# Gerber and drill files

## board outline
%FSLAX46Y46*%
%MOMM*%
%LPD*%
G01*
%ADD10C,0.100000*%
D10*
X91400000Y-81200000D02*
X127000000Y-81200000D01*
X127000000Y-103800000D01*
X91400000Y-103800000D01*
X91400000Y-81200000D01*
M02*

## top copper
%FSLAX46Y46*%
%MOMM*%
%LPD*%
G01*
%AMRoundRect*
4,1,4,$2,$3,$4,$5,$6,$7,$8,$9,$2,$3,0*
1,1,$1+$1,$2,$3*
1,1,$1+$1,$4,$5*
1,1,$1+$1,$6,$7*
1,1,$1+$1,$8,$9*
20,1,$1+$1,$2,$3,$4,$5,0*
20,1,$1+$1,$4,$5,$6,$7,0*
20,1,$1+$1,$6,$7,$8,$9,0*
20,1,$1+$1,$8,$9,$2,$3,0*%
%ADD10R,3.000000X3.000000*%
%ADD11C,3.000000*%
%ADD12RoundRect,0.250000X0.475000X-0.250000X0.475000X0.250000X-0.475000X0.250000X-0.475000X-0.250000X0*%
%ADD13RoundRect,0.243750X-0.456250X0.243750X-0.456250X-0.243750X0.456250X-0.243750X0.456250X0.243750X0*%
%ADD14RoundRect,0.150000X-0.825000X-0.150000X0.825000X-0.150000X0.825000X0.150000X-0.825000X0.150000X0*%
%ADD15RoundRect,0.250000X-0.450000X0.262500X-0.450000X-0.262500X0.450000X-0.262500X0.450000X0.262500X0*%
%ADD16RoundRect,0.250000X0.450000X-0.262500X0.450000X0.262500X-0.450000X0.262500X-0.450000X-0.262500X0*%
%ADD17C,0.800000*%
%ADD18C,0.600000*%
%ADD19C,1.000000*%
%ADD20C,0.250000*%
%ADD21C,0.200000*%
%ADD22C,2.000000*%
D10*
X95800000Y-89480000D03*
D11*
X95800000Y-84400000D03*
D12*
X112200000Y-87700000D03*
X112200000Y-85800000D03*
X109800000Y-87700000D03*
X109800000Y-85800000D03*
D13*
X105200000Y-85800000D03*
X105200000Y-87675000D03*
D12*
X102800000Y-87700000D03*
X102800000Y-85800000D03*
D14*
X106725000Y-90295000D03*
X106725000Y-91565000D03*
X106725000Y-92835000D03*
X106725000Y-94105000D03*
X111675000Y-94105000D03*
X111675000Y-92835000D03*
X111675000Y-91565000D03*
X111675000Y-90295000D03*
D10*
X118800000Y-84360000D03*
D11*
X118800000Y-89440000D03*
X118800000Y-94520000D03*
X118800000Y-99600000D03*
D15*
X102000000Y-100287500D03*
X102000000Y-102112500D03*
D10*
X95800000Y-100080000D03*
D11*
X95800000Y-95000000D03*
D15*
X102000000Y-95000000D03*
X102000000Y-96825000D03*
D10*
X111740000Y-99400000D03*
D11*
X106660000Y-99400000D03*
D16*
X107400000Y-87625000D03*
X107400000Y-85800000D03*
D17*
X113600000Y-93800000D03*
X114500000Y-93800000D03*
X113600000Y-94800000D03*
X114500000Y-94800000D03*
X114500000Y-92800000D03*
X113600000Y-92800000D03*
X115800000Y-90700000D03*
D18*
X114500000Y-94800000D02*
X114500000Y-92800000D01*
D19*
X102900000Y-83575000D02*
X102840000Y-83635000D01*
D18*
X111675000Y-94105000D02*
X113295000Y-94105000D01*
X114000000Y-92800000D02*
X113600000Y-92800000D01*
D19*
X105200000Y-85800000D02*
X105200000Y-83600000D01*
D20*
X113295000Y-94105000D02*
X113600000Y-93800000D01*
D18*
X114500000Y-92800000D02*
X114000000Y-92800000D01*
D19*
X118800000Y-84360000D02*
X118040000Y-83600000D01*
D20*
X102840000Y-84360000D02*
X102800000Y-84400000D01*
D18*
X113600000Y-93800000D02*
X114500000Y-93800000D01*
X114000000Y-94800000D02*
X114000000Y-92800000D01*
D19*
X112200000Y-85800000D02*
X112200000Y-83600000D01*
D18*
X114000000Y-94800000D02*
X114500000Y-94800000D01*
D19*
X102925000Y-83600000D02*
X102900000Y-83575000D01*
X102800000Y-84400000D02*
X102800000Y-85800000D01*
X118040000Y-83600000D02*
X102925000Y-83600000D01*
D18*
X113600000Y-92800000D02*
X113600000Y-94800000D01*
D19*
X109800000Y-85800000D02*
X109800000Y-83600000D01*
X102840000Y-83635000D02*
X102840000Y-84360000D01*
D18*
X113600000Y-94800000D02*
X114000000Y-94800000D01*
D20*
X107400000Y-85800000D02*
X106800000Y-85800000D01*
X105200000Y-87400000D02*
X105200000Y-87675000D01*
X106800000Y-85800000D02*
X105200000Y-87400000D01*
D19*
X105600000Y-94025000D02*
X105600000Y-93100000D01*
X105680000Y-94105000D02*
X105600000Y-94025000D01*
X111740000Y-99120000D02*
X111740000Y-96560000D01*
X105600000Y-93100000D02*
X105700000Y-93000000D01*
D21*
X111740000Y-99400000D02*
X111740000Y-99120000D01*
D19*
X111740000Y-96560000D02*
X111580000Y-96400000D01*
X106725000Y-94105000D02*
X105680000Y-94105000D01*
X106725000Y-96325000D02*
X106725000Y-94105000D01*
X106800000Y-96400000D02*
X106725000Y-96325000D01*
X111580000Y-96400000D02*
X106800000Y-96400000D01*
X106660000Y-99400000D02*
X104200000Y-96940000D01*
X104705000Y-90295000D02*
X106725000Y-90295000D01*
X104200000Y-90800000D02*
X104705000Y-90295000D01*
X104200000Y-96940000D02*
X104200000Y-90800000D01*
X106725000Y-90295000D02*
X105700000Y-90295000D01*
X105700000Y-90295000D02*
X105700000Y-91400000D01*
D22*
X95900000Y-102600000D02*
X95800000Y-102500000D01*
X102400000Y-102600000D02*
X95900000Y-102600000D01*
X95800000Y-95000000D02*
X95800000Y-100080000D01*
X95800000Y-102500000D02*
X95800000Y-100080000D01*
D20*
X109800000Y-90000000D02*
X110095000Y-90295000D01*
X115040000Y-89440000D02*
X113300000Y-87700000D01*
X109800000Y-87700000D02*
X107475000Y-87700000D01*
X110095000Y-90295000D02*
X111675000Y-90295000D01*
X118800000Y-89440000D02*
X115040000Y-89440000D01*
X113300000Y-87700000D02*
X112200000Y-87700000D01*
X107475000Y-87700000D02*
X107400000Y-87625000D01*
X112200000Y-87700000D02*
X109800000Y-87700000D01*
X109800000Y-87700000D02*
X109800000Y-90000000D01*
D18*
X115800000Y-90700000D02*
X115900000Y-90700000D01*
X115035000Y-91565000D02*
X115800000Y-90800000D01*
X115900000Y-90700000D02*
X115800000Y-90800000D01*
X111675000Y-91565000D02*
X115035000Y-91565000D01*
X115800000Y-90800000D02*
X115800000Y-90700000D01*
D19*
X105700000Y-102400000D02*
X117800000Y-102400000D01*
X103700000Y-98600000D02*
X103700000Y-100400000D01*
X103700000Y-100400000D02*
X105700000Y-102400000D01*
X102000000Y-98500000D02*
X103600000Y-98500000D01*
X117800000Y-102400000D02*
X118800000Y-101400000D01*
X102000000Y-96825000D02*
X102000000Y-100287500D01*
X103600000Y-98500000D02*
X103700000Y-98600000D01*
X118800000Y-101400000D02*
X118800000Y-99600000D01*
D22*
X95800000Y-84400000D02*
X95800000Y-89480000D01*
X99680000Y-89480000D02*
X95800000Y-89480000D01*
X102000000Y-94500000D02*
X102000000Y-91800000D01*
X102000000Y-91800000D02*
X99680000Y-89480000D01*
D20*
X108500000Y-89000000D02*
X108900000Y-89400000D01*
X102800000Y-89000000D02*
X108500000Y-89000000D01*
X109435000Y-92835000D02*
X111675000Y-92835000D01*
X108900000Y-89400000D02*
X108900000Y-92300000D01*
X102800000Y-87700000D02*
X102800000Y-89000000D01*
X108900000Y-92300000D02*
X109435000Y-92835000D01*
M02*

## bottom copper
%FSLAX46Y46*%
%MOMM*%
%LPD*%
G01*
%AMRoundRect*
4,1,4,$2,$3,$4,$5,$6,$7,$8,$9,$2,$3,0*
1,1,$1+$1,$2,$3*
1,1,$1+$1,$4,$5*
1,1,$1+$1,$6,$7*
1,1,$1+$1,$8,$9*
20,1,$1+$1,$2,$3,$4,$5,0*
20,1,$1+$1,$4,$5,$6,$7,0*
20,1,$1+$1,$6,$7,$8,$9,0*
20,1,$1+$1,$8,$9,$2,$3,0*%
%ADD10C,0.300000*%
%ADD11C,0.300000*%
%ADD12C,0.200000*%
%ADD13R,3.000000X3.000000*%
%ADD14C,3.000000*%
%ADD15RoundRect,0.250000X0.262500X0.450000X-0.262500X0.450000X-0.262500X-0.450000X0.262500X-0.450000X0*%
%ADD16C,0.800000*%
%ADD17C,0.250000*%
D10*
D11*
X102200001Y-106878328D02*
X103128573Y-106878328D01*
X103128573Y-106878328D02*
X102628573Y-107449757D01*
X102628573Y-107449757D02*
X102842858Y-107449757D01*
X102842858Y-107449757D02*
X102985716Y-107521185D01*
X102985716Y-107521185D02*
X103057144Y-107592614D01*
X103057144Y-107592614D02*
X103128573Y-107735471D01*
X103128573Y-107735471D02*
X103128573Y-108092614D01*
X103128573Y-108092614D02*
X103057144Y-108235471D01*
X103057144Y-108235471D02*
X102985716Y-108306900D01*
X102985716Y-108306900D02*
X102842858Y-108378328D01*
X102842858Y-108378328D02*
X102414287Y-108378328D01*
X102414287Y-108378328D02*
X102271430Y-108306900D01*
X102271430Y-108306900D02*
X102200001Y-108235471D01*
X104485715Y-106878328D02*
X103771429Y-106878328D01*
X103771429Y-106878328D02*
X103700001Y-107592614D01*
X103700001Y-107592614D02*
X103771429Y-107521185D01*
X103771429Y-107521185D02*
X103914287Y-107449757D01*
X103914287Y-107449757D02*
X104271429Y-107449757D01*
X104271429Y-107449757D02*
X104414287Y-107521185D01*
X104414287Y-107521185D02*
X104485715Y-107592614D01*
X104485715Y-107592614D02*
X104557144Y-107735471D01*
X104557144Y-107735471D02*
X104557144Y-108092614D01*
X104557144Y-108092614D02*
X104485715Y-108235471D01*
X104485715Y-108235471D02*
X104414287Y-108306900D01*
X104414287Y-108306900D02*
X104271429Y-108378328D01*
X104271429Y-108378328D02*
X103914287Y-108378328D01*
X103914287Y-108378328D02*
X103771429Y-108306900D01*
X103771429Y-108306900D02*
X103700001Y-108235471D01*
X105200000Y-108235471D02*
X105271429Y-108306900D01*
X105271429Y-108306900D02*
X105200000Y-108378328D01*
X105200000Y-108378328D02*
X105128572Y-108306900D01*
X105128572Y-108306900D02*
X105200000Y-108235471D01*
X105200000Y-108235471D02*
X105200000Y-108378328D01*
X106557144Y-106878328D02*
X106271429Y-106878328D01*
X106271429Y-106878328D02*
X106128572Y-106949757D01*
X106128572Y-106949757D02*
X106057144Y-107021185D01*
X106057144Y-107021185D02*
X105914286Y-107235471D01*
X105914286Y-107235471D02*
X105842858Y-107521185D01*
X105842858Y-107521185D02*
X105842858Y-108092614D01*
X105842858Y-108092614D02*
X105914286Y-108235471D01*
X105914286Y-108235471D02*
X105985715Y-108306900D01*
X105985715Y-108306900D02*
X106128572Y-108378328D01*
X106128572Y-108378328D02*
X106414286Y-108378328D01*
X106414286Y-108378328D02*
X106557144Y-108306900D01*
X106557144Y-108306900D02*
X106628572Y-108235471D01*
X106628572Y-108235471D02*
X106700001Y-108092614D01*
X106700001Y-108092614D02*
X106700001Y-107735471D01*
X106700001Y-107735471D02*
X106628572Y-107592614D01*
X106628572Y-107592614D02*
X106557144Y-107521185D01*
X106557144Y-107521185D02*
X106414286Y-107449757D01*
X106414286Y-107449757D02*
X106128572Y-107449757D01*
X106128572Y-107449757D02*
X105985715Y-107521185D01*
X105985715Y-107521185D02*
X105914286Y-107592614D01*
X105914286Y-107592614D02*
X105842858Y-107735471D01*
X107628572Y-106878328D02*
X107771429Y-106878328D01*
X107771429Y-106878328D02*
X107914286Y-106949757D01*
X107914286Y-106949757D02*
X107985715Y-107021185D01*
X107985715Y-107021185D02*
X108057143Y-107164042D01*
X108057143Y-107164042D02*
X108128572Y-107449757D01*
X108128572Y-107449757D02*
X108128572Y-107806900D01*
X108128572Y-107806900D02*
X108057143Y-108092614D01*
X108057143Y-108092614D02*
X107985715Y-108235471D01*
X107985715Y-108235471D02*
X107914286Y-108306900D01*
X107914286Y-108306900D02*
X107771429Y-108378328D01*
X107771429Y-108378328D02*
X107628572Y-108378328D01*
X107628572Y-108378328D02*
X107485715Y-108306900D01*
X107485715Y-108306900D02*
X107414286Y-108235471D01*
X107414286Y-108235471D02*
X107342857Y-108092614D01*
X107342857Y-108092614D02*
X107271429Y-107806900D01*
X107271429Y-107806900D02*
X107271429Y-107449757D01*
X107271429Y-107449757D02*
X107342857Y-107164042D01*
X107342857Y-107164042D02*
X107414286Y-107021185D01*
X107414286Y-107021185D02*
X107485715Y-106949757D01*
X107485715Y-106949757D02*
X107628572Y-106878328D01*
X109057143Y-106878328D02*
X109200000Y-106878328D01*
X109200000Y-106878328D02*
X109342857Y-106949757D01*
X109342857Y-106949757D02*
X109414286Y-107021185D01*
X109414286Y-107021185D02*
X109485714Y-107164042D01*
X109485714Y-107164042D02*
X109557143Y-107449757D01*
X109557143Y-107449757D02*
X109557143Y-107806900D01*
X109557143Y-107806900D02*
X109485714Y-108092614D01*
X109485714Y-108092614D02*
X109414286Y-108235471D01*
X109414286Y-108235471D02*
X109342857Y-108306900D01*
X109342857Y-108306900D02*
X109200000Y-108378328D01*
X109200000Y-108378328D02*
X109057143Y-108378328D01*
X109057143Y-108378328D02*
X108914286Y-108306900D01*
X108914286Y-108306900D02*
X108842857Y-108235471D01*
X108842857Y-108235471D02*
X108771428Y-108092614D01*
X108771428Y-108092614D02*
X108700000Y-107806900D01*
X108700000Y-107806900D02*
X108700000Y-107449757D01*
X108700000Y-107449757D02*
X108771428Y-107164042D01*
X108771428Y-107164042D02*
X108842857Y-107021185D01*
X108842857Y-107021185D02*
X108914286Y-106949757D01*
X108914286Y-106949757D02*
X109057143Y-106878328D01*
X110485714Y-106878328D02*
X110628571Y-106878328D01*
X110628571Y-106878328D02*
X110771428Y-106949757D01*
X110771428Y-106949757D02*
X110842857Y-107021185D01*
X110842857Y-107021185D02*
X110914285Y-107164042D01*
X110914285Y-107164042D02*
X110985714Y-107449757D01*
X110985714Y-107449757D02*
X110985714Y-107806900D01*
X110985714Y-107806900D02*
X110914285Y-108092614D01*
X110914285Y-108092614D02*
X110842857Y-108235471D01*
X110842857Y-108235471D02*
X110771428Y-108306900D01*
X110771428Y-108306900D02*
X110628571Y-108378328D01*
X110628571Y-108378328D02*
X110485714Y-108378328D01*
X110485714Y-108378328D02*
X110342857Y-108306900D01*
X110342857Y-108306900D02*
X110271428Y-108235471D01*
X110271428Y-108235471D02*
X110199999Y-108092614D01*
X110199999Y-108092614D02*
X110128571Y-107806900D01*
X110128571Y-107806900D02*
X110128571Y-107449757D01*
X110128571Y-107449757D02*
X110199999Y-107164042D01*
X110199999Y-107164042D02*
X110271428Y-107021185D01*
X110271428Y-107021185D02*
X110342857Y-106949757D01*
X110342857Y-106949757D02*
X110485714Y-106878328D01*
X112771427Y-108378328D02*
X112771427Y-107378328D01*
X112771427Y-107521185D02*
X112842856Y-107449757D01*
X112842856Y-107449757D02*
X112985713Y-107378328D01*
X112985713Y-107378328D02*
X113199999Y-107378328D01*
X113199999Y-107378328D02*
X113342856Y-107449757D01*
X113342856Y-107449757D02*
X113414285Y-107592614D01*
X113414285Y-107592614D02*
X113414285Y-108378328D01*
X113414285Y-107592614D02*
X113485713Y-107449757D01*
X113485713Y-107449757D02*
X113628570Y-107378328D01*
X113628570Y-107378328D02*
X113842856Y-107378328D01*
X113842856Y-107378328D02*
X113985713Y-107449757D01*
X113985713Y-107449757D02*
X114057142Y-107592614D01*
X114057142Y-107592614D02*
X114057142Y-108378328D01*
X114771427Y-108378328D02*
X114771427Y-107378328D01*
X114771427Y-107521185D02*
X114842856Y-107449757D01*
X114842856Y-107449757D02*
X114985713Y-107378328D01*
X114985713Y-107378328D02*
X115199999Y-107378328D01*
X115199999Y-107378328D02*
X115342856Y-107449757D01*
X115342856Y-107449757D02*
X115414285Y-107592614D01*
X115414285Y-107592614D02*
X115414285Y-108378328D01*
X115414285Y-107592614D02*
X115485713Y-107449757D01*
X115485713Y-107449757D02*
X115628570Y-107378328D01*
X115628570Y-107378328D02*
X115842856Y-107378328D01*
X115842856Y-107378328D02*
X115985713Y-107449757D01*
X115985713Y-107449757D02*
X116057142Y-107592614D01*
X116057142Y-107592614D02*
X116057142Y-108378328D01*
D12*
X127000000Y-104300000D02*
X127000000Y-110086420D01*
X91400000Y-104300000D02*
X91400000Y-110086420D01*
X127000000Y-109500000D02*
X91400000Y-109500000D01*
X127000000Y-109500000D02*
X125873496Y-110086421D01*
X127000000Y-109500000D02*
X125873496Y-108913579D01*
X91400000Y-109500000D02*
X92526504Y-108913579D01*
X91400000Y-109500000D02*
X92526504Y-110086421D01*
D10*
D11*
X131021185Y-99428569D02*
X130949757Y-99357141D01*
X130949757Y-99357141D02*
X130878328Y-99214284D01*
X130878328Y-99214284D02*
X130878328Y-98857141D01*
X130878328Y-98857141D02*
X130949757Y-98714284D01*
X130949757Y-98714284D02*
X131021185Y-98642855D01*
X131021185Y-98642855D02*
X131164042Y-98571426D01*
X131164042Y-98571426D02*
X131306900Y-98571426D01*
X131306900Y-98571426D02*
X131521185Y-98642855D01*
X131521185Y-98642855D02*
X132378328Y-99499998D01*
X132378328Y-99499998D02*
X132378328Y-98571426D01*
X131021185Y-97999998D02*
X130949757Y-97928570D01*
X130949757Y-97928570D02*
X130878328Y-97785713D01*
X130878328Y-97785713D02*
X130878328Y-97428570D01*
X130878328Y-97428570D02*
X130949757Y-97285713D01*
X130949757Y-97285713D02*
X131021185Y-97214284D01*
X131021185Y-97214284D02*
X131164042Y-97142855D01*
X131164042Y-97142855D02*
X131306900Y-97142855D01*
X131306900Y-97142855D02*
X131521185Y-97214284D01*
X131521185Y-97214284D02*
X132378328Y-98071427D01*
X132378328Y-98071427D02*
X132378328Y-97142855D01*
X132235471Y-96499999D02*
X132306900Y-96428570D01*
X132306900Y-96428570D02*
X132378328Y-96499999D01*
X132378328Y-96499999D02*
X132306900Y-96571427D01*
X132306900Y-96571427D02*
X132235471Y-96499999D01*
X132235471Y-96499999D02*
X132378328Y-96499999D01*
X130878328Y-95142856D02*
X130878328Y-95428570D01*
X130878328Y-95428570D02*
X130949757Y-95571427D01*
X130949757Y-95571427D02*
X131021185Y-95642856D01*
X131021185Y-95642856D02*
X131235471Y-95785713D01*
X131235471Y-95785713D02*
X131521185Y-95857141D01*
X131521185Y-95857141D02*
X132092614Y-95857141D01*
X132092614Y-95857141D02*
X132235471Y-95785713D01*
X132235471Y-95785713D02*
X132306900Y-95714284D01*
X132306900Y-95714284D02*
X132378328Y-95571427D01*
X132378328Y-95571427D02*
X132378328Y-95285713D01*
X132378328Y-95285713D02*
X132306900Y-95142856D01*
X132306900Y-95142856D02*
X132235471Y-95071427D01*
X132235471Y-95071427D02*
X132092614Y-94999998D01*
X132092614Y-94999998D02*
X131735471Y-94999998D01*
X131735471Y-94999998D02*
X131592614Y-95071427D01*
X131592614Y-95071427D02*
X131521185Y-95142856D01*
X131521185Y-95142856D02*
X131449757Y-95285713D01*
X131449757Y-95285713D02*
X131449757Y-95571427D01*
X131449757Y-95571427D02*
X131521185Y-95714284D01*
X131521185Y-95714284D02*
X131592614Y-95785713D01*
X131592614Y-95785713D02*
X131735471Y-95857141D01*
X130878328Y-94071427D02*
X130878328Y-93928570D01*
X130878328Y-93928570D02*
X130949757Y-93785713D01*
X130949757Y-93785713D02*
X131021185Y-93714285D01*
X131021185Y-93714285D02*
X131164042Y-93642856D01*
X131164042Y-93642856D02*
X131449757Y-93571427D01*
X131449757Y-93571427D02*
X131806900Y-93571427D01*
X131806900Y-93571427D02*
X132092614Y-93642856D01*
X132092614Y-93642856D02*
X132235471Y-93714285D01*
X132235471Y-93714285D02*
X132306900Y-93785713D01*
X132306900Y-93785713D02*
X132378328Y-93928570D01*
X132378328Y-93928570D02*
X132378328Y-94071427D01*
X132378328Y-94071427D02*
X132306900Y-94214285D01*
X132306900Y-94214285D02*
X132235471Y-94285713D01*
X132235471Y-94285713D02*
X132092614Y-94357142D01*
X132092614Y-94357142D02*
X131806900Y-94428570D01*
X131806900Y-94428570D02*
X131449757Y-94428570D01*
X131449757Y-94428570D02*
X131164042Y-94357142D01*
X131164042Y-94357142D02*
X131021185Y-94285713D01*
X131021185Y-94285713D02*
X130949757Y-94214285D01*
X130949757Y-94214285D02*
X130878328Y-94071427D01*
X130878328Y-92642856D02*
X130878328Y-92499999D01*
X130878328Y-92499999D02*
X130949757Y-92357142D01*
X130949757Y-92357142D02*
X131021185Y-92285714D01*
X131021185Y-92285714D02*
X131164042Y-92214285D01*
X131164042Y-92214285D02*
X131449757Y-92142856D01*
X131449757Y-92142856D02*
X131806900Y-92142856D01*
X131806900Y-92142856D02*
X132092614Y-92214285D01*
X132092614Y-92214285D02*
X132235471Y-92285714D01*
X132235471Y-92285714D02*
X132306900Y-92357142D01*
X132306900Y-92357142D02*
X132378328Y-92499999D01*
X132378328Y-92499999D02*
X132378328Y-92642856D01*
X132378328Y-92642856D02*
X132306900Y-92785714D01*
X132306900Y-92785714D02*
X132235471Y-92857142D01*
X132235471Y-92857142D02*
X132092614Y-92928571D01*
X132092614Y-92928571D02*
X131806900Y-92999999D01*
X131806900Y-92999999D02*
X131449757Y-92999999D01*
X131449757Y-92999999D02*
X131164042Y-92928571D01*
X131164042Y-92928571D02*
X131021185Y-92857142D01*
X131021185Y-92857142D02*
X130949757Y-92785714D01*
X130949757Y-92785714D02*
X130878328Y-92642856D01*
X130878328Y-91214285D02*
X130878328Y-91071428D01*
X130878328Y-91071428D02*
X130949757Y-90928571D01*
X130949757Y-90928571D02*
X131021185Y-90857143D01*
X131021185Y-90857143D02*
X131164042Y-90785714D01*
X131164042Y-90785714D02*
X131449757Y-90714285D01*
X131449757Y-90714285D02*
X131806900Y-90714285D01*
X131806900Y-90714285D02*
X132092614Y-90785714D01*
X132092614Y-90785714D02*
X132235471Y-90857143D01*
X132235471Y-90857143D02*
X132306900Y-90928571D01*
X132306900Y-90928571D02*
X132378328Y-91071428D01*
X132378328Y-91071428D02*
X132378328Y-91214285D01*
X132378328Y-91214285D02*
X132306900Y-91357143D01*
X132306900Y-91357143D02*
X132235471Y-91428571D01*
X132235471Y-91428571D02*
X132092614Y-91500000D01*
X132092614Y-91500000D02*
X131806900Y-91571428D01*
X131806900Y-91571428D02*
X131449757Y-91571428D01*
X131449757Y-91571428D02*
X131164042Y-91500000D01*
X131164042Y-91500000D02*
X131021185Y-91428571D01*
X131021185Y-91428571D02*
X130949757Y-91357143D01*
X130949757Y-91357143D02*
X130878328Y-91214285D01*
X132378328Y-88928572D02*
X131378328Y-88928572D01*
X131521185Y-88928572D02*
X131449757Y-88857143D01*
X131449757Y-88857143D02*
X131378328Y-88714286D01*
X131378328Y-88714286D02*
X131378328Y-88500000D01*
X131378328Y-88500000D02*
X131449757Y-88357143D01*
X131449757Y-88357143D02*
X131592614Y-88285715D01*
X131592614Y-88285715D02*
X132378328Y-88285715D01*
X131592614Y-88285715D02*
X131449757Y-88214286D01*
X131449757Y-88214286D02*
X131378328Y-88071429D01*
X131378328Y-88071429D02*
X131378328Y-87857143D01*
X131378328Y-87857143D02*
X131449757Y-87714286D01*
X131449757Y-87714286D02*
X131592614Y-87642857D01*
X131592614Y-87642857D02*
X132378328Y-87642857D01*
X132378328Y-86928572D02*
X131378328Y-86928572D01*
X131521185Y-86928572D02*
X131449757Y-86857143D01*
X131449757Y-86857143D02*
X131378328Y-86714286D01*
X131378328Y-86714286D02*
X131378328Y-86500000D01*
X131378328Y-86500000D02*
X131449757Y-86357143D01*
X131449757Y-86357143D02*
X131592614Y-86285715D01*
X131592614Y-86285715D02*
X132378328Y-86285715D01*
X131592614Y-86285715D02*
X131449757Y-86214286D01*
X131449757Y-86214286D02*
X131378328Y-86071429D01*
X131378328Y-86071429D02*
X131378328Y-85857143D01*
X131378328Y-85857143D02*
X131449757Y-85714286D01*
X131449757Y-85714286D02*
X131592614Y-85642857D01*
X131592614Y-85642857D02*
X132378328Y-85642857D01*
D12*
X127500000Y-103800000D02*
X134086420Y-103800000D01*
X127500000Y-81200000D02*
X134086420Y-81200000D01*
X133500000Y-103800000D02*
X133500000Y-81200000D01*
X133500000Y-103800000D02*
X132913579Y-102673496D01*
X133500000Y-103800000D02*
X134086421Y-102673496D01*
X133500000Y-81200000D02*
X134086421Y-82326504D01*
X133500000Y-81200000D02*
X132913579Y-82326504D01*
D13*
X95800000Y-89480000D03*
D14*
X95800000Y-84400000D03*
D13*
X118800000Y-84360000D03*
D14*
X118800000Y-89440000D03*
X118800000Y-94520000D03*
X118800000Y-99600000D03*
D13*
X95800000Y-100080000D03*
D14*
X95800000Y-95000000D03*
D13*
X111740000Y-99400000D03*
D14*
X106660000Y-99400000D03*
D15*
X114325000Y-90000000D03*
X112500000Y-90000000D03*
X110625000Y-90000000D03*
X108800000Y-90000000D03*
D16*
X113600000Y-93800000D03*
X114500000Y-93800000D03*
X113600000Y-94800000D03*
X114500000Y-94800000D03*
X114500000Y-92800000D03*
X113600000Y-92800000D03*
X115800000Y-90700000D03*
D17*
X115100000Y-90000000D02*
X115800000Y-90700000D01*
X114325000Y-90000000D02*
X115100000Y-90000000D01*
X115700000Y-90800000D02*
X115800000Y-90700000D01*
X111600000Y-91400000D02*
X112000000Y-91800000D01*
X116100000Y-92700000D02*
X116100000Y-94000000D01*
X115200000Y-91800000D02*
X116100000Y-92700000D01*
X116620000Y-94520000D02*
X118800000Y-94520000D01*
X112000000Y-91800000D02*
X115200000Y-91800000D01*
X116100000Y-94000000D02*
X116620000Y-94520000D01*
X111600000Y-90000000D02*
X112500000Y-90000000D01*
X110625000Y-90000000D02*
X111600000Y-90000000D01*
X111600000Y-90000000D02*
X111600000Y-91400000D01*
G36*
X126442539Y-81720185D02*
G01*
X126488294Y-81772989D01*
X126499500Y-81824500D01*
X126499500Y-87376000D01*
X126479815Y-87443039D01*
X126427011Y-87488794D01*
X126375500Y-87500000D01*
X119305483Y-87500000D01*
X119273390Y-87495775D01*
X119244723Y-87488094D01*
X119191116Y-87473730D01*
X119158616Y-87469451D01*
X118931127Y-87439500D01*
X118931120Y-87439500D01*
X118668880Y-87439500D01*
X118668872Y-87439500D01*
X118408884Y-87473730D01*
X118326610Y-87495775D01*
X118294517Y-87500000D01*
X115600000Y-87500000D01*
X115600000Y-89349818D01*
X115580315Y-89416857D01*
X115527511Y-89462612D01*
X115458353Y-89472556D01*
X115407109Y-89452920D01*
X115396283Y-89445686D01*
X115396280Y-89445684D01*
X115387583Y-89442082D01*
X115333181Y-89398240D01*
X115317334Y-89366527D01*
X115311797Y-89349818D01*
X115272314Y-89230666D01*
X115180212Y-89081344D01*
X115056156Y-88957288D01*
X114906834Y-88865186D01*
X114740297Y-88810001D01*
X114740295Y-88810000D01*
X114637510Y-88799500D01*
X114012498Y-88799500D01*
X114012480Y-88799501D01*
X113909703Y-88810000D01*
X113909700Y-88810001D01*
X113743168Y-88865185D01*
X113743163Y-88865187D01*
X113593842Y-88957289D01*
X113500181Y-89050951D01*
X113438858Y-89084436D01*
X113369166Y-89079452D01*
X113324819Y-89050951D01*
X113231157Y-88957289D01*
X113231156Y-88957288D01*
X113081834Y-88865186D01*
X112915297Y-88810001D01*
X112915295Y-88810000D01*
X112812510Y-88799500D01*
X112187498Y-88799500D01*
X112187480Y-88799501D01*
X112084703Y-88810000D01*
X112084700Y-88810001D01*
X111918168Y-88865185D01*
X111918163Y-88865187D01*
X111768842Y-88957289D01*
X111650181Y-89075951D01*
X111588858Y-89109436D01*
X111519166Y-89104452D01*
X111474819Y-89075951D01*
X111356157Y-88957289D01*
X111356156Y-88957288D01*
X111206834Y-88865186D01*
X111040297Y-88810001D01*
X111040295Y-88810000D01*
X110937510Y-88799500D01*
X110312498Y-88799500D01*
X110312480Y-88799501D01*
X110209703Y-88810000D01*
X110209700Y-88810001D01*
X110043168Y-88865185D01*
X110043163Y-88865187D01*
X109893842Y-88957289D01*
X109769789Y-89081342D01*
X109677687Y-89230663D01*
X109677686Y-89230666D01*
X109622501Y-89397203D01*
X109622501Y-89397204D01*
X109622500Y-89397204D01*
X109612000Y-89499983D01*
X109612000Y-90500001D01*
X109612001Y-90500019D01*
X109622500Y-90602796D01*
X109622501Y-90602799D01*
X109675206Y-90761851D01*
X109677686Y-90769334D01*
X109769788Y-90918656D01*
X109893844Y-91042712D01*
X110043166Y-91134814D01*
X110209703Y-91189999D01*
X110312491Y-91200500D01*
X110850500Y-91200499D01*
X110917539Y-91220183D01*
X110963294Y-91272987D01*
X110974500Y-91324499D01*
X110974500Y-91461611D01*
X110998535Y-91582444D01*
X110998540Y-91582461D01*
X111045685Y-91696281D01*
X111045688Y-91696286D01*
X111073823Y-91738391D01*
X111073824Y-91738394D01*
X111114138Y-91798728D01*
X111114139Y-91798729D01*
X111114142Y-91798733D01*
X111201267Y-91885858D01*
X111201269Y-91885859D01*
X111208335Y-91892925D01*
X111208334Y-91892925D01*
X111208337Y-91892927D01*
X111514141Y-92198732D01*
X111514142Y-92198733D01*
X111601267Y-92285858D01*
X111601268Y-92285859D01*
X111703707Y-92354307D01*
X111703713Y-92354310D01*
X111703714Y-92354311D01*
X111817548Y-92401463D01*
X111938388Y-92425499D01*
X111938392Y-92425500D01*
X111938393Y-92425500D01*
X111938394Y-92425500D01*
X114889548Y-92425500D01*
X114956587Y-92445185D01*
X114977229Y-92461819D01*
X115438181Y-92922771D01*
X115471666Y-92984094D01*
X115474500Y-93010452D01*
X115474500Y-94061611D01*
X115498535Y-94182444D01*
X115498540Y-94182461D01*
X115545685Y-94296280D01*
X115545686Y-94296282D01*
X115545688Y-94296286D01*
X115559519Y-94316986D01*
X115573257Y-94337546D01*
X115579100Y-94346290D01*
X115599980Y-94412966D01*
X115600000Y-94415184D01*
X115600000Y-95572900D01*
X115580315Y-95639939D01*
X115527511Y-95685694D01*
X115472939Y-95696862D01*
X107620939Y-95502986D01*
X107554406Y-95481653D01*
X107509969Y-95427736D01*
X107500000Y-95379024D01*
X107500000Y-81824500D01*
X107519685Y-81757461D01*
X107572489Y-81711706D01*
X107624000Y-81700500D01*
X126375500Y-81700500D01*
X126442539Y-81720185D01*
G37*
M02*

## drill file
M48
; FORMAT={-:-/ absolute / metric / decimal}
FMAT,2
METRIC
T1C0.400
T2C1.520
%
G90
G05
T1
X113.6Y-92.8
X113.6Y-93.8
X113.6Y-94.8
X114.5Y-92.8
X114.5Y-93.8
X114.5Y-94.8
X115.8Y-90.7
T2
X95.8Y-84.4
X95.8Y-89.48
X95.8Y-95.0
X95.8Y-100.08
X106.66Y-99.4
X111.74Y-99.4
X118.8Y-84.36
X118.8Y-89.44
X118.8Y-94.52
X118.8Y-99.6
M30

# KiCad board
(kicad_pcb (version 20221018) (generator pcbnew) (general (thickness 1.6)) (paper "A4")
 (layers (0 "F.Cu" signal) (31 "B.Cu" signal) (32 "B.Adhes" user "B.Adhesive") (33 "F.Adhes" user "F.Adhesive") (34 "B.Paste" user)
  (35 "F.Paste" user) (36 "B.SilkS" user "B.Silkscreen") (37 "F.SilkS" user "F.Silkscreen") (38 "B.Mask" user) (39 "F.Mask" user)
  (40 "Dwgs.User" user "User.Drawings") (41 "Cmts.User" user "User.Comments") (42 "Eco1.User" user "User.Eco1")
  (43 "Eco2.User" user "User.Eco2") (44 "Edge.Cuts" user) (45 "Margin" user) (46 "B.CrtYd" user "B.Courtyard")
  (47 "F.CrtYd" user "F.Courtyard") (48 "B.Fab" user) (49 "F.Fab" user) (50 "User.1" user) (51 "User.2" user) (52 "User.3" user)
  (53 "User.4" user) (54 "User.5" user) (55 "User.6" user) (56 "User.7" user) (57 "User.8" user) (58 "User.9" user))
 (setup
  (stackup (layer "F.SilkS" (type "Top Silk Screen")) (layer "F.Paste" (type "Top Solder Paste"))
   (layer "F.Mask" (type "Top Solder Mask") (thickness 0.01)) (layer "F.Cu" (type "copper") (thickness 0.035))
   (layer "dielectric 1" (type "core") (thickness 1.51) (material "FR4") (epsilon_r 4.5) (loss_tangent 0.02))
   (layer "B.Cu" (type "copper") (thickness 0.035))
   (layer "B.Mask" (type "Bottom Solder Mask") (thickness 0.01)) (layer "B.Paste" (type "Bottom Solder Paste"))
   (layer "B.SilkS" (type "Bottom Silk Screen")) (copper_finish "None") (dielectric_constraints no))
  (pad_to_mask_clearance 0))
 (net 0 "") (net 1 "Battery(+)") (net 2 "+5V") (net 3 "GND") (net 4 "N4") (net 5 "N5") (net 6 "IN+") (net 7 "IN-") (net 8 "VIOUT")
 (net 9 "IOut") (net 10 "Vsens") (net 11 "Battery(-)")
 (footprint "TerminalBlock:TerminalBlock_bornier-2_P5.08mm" (layer "F.Cu") (at 95.8 89.48 90)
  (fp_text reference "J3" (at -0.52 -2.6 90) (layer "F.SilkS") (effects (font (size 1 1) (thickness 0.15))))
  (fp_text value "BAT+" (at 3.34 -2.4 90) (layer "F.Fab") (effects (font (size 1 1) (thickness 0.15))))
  (pad "1" thru_hole rect (at 0 0 90) (size 3 3) (drill 1.52) (layers "*.Cu" "*.Mask") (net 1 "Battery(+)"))
  (pad "2" thru_hole circle (at 5.08 0 90) (size 3 3) (drill 1.52) (layers "*.Cu" "*.Mask") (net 1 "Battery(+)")))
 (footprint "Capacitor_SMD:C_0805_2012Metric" (layer "F.Cu") (at 112.2 86.75 90)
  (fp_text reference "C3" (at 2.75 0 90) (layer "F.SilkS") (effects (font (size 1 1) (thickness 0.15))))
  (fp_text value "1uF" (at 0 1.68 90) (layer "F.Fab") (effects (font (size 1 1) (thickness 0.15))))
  (pad "1" smd roundrect (at -0.95 0 90) (size 1 1.45) (layers "F.Cu" "F.Paste" "F.Mask") (roundrect_rratio 0.25) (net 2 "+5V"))
  (pad "2" smd roundrect (at 0.95 0 90) (size 1 1.45) (layers "F.Cu" "F.Paste" "F.Mask") (roundrect_rratio 0.25) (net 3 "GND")))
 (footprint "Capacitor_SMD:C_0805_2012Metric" (layer "F.Cu") (at 109.8 86.75 90)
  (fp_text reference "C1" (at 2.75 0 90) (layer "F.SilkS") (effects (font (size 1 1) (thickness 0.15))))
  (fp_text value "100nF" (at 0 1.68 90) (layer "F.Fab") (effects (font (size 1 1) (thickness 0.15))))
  (pad "1" smd roundrect (at -0.95 0 90) (size 1 1.45) (layers "F.Cu" "F.Paste" "F.Mask") (roundrect_rratio 0.25) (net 2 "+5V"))
  (pad "2" smd roundrect (at 0.95 0 90) (size 1 1.45) (layers "F.Cu" "F.Paste" "F.Mask") (roundrect_rratio 0.25) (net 3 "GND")))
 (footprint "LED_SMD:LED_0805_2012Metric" (layer "F.Cu") (at 105.2 86.7375 -90)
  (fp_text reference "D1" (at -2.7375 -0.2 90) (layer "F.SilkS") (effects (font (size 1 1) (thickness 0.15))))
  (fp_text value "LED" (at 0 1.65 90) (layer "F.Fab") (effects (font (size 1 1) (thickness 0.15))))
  (pad "1" smd roundrect (at -0.9375 0 270) (size 0.975 1.4) (layers "F.Cu" "F.Paste" "F.Mask") (roundrect_rratio 0.25) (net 3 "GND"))
  (pad "2" smd roundrect (at 0.9375 0 270) (size 0.975 1.4) (layers "F.Cu" "F.Paste" "F.Mask") (roundrect_rratio 0.25) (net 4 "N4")))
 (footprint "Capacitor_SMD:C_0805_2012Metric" (layer "F.Cu") (at 102.8 86.75 90)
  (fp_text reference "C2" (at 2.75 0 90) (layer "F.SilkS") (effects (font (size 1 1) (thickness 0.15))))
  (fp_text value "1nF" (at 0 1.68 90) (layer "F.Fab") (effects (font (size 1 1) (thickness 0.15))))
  (pad "1" smd roundrect (at -0.95 0 90) (size 1 1.45) (layers "F.Cu" "F.Paste" "F.Mask") (roundrect_rratio 0.25) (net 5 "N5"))
  (pad "2" smd roundrect (at 0.95 0 90) (size 1 1.45) (layers "F.Cu" "F.Paste" "F.Mask") (roundrect_rratio 0.25) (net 3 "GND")))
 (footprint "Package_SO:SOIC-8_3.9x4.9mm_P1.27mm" (layer "F.Cu") (at 109.2 92.2)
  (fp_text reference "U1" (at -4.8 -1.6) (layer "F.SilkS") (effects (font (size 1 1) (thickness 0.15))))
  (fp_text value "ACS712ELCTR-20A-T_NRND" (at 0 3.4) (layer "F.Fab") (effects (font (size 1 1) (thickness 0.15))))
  (pad "1" smd roundrect (at -2.475 -1.905) (size 1.95 0.6) (layers "F.Cu" "F.Paste" "F.Mask") (roundrect_rratio 0.25) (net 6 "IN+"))
  (pad "2" smd roundrect (at -2.475 -0.635) (size 1.95 0.6) (layers "F.Cu" "F.Paste" "F.Mask") (roundrect_rratio 0.25) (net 6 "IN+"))
  (pad "3" smd roundrect (at -2.475 0.635) (size 1.95 0.6) (layers "F.Cu" "F.Paste" "F.Mask") (roundrect_rratio 0.25) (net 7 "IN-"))
  (pad "4" smd roundrect (at -2.475 1.905) (size 1.95 0.6) (layers "F.Cu" "F.Paste" "F.Mask") (roundrect_rratio 0.25) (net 7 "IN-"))
  (pad "5" smd roundrect (at 2.475 1.905) (size 1.95 0.6) (layers "F.Cu" "F.Paste" "F.Mask") (roundrect_rratio 0.25) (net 3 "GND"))
  (pad "6" smd roundrect (at 2.475 0.635) (size 1.95 0.6) (layers "F.Cu" "F.Paste" "F.Mask") (roundrect_rratio 0.25) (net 5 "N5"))
  (pad "7" smd roundrect (at 2.475 -0.635) (size 1.95 0.6) (layers "F.Cu" "F.Paste" "F.Mask") (roundrect_rratio 0.25) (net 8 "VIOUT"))
  (pad "8" smd roundrect (at 2.475 -1.905) (size 1.95 0.6) (layers "F.Cu" "F.Paste" "F.Mask") (roundrect_rratio 0.25) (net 2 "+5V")))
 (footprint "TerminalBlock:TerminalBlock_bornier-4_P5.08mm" (layer "F.Cu") (at 118.8 84.36 -90)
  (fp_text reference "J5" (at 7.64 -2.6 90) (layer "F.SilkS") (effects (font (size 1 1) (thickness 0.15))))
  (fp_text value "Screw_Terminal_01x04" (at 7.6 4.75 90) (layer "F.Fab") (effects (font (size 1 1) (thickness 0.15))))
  (pad "1" thru_hole rect (at 0 0 270) (size 3 3) (drill 1.52) (layers "*.Cu" "*.Mask") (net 3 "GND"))
  (pad "2" thru_hole circle (at 5.08 0 270) (size 3 3) (drill 1.52) (layers "*.Cu" "*.Mask") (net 2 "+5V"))
  (pad "3" thru_hole circle (at 10.16 0 270) (size 3 3) (drill 1.52) (layers "*.Cu" "*.Mask") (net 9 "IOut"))
  (pad "4" thru_hole circle (at 15.24 0 270) (size 3 3) (drill 1.52) (layers "*.Cu" "*.Mask") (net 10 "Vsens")))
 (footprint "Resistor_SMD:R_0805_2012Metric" (layer "F.Cu") (at 102 101.2 -90)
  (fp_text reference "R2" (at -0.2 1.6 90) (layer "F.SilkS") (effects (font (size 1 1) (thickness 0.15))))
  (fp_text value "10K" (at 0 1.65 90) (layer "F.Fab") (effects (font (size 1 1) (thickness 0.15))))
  (pad "1" smd roundrect (at -0.9125 0 270) (size 1.025 1.4) (layers "F.Cu" "F.Paste" "F.Mask") (roundrect_rratio 0.243902439)
   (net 10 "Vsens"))
  (pad "2" smd roundrect (at 0.9125 0 270) (size 1.025 1.4) (layers "F.Cu" "F.Paste" "F.Mask") (roundrect_rratio 0.243902439)
   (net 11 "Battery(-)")))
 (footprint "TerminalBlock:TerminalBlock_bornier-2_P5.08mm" (layer "F.Cu") (at 95.8 100.08 90)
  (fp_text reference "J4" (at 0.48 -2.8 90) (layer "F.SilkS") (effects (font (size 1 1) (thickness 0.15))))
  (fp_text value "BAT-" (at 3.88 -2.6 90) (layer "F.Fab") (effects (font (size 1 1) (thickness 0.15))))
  (pad "1" thru_hole rect (at 0 0 90) (size 3 3) (drill 1.52) (layers "*.Cu" "*.Mask") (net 11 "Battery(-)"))
  (pad "2" thru_hole circle (at 5.08 0 90) (size 3 3) (drill 1.52) (layers "*.Cu" "*.Mask") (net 11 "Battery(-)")))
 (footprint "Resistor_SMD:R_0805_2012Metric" (layer "F.Cu") (at 102 95.9125 -90)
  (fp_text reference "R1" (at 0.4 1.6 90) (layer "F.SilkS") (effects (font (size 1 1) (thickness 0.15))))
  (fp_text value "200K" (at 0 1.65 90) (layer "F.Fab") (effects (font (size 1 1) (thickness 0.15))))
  (pad "1" smd roundrect (at -0.9125 0 270) (size 1.025 1.4) (layers "F.Cu" "F.Paste" "F.Mask") (roundrect_rratio 0.243902439)
   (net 1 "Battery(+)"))
  (pad "2" smd roundrect (at 0.9125 0 270) (size 1.025 1.4) (layers "F.Cu" "F.Paste" "F.Mask") (roundrect_rratio 0.243902439)
   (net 10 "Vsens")))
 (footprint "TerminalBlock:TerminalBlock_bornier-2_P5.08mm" (layer "F.Cu") (at 111.74 99.4 180)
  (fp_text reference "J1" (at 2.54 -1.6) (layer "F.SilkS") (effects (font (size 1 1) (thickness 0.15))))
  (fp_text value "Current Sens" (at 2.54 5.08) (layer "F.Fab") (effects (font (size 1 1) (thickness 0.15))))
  (pad "1" thru_hole rect (at 0 0 180) (size 3 3) (drill 1.52) (layers "*.Cu" "*.Mask") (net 7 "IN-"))
  (pad "2" thru_hole circle (at 5.08 0 180) (size 3 3) (drill 1.52) (layers "*.Cu" "*.Mask") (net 6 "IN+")))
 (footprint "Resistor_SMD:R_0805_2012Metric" (layer "F.Cu") (at 107.4 86.7125 90)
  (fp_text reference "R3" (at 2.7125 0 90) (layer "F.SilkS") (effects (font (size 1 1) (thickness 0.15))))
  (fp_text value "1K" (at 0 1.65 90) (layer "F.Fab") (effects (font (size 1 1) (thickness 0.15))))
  (pad "1" smd roundrect (at -0.9125 0 90) (size 1.025 1.4) (layers "F.Cu" "F.Paste" "F.Mask") (roundrect_rratio 0.243902439) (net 2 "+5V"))
  (pad "2" smd roundrect (at 0.9125 0 90) (size 1.025 1.4) (layers "F.Cu" "F.Paste" "F.Mask") (roundrect_rratio 0.243902439) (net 4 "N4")))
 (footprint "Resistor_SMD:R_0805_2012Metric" (layer "B.Cu") (at 113.4125 90 180)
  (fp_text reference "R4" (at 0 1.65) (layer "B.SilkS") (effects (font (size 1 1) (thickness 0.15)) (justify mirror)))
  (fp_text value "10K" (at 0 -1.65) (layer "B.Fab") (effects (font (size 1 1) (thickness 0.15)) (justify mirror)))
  (pad "1" smd roundrect (at -0.9125 0 180) (size 1.025 1.4) (layers "B.Cu" "B.Paste" "B.Mask") (roundrect_rratio 0.243902439)
   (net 8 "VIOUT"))
  (pad "2" smd roundrect (at 0.9125 0 180) (size 1.025 1.4) (layers "B.Cu" "B.Paste" "B.Mask") (roundrect_rratio 0.243902439) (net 9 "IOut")))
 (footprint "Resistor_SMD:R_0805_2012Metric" (layer "B.Cu") (at 109.7125 90 180)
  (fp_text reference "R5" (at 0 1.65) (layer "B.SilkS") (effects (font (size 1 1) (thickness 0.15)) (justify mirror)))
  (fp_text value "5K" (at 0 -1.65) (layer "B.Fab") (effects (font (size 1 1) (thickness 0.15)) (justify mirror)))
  (pad "1" smd roundrect (at -0.9125 0 180) (size 1.025 1.4) (layers "B.Cu" "B.Paste" "B.Mask") (roundrect_rratio 0.243902439)
   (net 9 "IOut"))
  (pad "2" smd roundrect (at 0.9125 0 180) (size 1.025 1.4) (layers "B.Cu" "B.Paste" "B.Mask") (roundrect_rratio 0.243902439) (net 3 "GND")))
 (gr_rect (start 91.4 81.2) (end 127 103.8) (stroke (width 0.1) (type default)) (fill none) (layer "Edge.Cuts"))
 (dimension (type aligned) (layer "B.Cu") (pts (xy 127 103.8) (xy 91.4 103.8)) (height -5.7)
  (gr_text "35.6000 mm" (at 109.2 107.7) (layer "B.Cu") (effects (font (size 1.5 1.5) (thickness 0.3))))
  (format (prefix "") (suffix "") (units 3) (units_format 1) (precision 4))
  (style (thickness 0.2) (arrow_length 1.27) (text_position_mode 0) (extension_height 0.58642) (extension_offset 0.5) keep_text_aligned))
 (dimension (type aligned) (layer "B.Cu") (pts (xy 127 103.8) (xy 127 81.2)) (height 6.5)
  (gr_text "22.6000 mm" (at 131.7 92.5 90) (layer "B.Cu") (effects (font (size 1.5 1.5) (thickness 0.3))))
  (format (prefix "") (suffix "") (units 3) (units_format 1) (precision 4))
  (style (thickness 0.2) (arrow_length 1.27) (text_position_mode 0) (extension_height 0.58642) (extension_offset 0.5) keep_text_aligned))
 (segment (start 114.5 94.8) (end 114.5 92.8) (width 0.6) (layer "F.Cu") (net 3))
 (segment (start 102.9 83.575) (end 102.84 83.635) (width 1) (layer "F.Cu") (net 3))
 (segment (start 111.675 94.105) (end 113.295 94.105) (width 0.6) (layer "F.Cu") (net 3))
 (segment (start 114 92.8) (end 113.6 92.8) (width 0.6) (layer "F.Cu") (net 3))
 (segment (start 105.2 85.8) (end 105.2 83.6) (width 1) (layer "F.Cu") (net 3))
 (segment (start 113.295 94.105) (end 113.6 93.8) (width 0.25) (layer "F.Cu") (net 3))
 (segment (start 114.5 92.8) (end 114 92.8) (width 0.6) (layer "F.Cu") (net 3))
 (segment (start 118.8 84.36) (end 118.04 83.6) (width 1) (layer "F.Cu") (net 3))
 (segment (start 102.84 84.36) (end 102.8 84.4) (width 0.25) (layer "F.Cu") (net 3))
 (segment (start 113.6 93.8) (end 114.5 93.8) (width 0.6) (layer "F.Cu") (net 3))
 (segment (start 114 94.8) (end 114 92.8) (width 0.6) (layer "F.Cu") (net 3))
 (segment (start 112.2 85.8) (end 112.2 83.6) (width 1) (layer "F.Cu") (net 3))
 (segment (start 114 94.8) (end 114.5 94.8) (width 0.6) (layer "F.Cu") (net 3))
 (segment (start 102.925 83.6) (end 102.9 83.575) (width 1) (layer "F.Cu") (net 3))
 (segment (start 102.8 84.4) (end 102.8 85.8) (width 1) (layer "F.Cu") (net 3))
 (segment (start 118.04 83.6) (end 102.925 83.6) (width 1) (layer "F.Cu") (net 3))
 (segment (start 113.6 92.8) (end 113.6 94.8) (width 0.6) (layer "F.Cu") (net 3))
 (segment (start 109.8 85.8) (end 109.8 83.6) (width 1) (layer "F.Cu") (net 3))
 (segment (start 102.84 83.635) (end 102.84 84.36) (width 1) (layer "F.Cu") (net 3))
 (segment (start 113.6 94.8) (end 114 94.8) (width 0.6) (layer "F.Cu") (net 3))
 (via (at 113.6 93.8) (size 0.8) (drill 0.4) (layers "F.Cu" "B.Cu") (free) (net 3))
 (via (at 114.5 93.8) (size 0.8) (drill 0.4) (layers "F.Cu" "B.Cu") (free) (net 3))
 (via (at 113.6 94.8) (size 0.8) (drill 0.4) (layers "F.Cu" "B.Cu") (free) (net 3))
 (via (at 114.5 94.8) (size 0.8) (drill 0.4) (layers "F.Cu" "B.Cu") (free) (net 3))
 (via (at 114.5 92.8) (size 0.8) (drill 0.4) (layers "F.Cu" "B.Cu") (free) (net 3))
 (via (at 113.6 92.8) (size 0.8) (drill 0.4) (layers "F.Cu" "B.Cu") (free) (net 3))
 (segment (start 107.4 85.8) (end 106.8 85.8) (width 0.25) (layer "F.Cu") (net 4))
 (segment (start 105.2 87.4) (end 105.2 87.675) (width 0.25) (layer "F.Cu") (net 4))
 (segment (start 106.8 85.8) (end 105.2 87.4) (width 0.25) (layer "F.Cu") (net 4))
 (segment (start 105.6 94.025) (end 105.6 93.1) (width 1) (layer "F.Cu") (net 7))
 (segment (start 105.68 94.105) (end 105.6 94.025) (width 1) (layer "F.Cu") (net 7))
 (segment (start 111.74 99.12) (end 111.74 96.56) (width 1) (layer "F.Cu") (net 7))
 (segment (start 105.6 93.1) (end 105.7 93) (width 1) (layer "F.Cu") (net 7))
 (segment (start 111.74 99.4) (end 111.74 99.12) (width 0.2) (layer "F.Cu") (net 7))
 (segment (start 111.74 96.56) (end 111.58 96.4) (width 1) (layer "F.Cu") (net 7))
 (segment (start 106.725 94.105) (end 105.68 94.105) (width 1) (layer "F.Cu") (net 7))
 (segment (start 106.725 96.325) (end 106.725 94.105) (width 1) (layer "F.Cu") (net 7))
 (segment (start 106.8 96.4) (end 106.725 96.325) (width 1) (layer "F.Cu") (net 7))
 (segment (start 111.58 96.4) (end 106.8 96.4) (width 1) (layer "F.Cu") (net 7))
 (segment (start 106.66 99.4) (end 104.2 96.94) (width 1) (layer "F.Cu") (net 6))
 (segment (start 104.705 90.295) (end 106.725 90.295) (width 1) (layer "F.Cu") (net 6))
 (segment (start 104.2 90.8) (end 104.705 90.295) (width 1) (layer "F.Cu") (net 6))
 (segment (start 104.2 96.94) (end 104.2 90.8) (width 1) (layer "F.Cu") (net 6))
 (segment (start 106.725 90.295) (end 105.7 90.295) (width 1) (layer "F.Cu") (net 6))
 (segment (start 105.7 90.295) (end 105.7 91.4) (width 1) (layer "F.Cu") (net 6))
 (segment (start 95.9 102.6) (end 95.8 102.5) (width 2) (layer "F.Cu") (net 11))
 (segment (start 102.4 102.6) (end 95.9 102.6) (width 2) (layer "F.Cu") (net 11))
 (segment (start 95.8 95) (end 95.8 100.08) (width 2) (layer "F.Cu") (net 11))
 (segment (start 95.8 102.5) (end 95.8 100.08) (width 2) (layer "F.Cu") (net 11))
 (segment (start 109.8 90) (end 110.095 90.295) (width 0.25) (layer "F.Cu") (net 2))
 (segment (start 115.04 89.44) (end 113.3 87.7) (width 0.25) (layer "F.Cu") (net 2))
 (segment (start 109.8 87.7) (end 107.475 87.7) (width 0.25) (layer "F.Cu") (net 2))
 (segment (start 110.095 90.295) (end 111.675 90.295) (width 0.25) (layer "F.Cu") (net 2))
 (segment (start 118.8 89.44) (end 115.04 89.44) (width 0.25) (layer "F.Cu") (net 2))
 (segment (start 113.3 87.7) (end 112.2 87.7) (width 0.25) (layer "F.Cu") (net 2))
 (segment (start 107.475 87.7) (end 107.4 87.625) (width 0.25) (layer "F.Cu") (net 2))
 (segment (start 112.2 87.7) (end 109.8 87.7) (width 0.25) (layer "F.Cu") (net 2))
 (segment (start 109.8 87.7) (end 109.8 90) (width 0.25) (layer "F.Cu") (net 2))
 (segment (start 115.8 90.7) (end 115.9 90.7) (width 0.6) (layer "F.Cu") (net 8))
 (segment (start 115.035 91.565) (end 115.8 90.8) (width 0.6) (layer "F.Cu") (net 8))
 (segment (start 115.9 90.7) (end 115.8 90.8) (width 0.6) (layer "F.Cu") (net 8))
 (segment (start 111.675 91.565) (end 115.035 91.565) (width 0.6) (layer "F.Cu") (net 8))
 (segment (start 115.8 90.8) (end 115.8 90.7) (width 0.6) (layer "F.Cu") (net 8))
 (via (at 115.8 90.7) (size 0.8) (drill 0.4) (layers "F.Cu" "B.Cu") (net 8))
 (segment (start 115.1 90) (end 115.8 90.7) (width 0.25) (layer "B.Cu") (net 8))
 (segment (start 114.325 90) (end 115.1 90) (width 0.25) (layer "B.Cu") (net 8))
 (segment (start 115.7 90.8) (end 115.8 90.7) (width 0.25) (layer "B.Cu") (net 8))
 (segment (start 105.7 102.4) (end 117.8 102.4) (width 1) (layer "F.Cu") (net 10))
 (segment (start 103.7 98.6) (end 103.7 100.4) (width 1) (layer "F.Cu") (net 10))
 (segment (start 103.7 100.4) (end 105.7 102.4) (width 1) (layer "F.Cu") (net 10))
 (segment (start 102 98.5) (end 103.6 98.5) (width 1) (layer "F.Cu") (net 10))
 (segment (start 117.8 102.4) (end 118.8 101.4) (width 1) (layer "F.Cu") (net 10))
 (segment (start 102 96.825) (end 102 100.2875) (width 1) (layer "F.Cu") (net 10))
 (segment (start 103.6 98.5) (end 103.7 98.6) (width 1) (layer "F.Cu") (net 10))
 (segment (start 118.8 101.4) (end 118.8 99.6) (width 1) (layer "F.Cu") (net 10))
 (segment (start 95.8 84.4) (end 95.8 89.48) (width 2) (layer "F.Cu") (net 1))
 (segment (start 99.68 89.48) (end 95.8 89.48) (width 2) (layer "F.Cu") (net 1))
 (segment (start 102 94.5) (end 102 91.8) (width 2) (layer "F.Cu") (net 1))
 (segment (start 102 91.8) (end 99.68 89.48) (width 2) (layer "F.Cu") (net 1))
 (segment (start 108.5 89) (end 108.9 89.4) (width 0.25) (layer "F.Cu") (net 5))
 (segment (start 102.8 89) (end 108.5 89) (width 0.25) (layer "F.Cu") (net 5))
 (segment (start 109.435 92.835) (end 111.675 92.835) (width 0.25) (layer "F.Cu") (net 5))
 (segment (start 108.9 89.4) (end 108.9 92.3) (width 0.25) (layer "F.Cu") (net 5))
 (segment (start 102.8 87.7) (end 102.8 89) (width 0.25) (layer "F.Cu") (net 5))
 (segment (start 108.9 92.3) (end 109.435 92.835) (width 0.25) (layer "F.Cu") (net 5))
 (segment (start 111.6 91.4) (end 112 91.8) (width 0.25) (layer "B.Cu") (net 9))
 (segment (start 116.1 92.7) (end 116.1 94) (width 0.25) (layer "B.Cu") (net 9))
 (segment (start 115.2 91.8) (end 116.1 92.7) (width 0.25) (layer "B.Cu") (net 9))
 (segment (start 116.62 94.52) (end 118.8 94.52) (width 0.25) (layer "B.Cu") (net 9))
 (segment (start 112 91.8) (end 115.2 91.8) (width 0.25) (layer "B.Cu") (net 9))
 (segment (start 116.1 94) (end 116.62 94.52) (width 0.25) (layer "B.Cu") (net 9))
 (segment (start 111.6 90) (end 112.5 90) (width 0.25) (layer "B.Cu") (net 9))
 (segment (start 110.625 90) (end 111.6 90) (width 0.25) (layer "B.Cu") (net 9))
 (segment (start 111.6 90) (end 111.6 91.4) (width 0.25) (layer "B.Cu") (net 9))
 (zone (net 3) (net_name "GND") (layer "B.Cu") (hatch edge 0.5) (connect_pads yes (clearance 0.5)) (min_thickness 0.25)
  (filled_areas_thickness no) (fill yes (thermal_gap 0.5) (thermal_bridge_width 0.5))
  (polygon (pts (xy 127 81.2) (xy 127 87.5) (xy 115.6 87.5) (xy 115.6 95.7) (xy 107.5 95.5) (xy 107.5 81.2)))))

